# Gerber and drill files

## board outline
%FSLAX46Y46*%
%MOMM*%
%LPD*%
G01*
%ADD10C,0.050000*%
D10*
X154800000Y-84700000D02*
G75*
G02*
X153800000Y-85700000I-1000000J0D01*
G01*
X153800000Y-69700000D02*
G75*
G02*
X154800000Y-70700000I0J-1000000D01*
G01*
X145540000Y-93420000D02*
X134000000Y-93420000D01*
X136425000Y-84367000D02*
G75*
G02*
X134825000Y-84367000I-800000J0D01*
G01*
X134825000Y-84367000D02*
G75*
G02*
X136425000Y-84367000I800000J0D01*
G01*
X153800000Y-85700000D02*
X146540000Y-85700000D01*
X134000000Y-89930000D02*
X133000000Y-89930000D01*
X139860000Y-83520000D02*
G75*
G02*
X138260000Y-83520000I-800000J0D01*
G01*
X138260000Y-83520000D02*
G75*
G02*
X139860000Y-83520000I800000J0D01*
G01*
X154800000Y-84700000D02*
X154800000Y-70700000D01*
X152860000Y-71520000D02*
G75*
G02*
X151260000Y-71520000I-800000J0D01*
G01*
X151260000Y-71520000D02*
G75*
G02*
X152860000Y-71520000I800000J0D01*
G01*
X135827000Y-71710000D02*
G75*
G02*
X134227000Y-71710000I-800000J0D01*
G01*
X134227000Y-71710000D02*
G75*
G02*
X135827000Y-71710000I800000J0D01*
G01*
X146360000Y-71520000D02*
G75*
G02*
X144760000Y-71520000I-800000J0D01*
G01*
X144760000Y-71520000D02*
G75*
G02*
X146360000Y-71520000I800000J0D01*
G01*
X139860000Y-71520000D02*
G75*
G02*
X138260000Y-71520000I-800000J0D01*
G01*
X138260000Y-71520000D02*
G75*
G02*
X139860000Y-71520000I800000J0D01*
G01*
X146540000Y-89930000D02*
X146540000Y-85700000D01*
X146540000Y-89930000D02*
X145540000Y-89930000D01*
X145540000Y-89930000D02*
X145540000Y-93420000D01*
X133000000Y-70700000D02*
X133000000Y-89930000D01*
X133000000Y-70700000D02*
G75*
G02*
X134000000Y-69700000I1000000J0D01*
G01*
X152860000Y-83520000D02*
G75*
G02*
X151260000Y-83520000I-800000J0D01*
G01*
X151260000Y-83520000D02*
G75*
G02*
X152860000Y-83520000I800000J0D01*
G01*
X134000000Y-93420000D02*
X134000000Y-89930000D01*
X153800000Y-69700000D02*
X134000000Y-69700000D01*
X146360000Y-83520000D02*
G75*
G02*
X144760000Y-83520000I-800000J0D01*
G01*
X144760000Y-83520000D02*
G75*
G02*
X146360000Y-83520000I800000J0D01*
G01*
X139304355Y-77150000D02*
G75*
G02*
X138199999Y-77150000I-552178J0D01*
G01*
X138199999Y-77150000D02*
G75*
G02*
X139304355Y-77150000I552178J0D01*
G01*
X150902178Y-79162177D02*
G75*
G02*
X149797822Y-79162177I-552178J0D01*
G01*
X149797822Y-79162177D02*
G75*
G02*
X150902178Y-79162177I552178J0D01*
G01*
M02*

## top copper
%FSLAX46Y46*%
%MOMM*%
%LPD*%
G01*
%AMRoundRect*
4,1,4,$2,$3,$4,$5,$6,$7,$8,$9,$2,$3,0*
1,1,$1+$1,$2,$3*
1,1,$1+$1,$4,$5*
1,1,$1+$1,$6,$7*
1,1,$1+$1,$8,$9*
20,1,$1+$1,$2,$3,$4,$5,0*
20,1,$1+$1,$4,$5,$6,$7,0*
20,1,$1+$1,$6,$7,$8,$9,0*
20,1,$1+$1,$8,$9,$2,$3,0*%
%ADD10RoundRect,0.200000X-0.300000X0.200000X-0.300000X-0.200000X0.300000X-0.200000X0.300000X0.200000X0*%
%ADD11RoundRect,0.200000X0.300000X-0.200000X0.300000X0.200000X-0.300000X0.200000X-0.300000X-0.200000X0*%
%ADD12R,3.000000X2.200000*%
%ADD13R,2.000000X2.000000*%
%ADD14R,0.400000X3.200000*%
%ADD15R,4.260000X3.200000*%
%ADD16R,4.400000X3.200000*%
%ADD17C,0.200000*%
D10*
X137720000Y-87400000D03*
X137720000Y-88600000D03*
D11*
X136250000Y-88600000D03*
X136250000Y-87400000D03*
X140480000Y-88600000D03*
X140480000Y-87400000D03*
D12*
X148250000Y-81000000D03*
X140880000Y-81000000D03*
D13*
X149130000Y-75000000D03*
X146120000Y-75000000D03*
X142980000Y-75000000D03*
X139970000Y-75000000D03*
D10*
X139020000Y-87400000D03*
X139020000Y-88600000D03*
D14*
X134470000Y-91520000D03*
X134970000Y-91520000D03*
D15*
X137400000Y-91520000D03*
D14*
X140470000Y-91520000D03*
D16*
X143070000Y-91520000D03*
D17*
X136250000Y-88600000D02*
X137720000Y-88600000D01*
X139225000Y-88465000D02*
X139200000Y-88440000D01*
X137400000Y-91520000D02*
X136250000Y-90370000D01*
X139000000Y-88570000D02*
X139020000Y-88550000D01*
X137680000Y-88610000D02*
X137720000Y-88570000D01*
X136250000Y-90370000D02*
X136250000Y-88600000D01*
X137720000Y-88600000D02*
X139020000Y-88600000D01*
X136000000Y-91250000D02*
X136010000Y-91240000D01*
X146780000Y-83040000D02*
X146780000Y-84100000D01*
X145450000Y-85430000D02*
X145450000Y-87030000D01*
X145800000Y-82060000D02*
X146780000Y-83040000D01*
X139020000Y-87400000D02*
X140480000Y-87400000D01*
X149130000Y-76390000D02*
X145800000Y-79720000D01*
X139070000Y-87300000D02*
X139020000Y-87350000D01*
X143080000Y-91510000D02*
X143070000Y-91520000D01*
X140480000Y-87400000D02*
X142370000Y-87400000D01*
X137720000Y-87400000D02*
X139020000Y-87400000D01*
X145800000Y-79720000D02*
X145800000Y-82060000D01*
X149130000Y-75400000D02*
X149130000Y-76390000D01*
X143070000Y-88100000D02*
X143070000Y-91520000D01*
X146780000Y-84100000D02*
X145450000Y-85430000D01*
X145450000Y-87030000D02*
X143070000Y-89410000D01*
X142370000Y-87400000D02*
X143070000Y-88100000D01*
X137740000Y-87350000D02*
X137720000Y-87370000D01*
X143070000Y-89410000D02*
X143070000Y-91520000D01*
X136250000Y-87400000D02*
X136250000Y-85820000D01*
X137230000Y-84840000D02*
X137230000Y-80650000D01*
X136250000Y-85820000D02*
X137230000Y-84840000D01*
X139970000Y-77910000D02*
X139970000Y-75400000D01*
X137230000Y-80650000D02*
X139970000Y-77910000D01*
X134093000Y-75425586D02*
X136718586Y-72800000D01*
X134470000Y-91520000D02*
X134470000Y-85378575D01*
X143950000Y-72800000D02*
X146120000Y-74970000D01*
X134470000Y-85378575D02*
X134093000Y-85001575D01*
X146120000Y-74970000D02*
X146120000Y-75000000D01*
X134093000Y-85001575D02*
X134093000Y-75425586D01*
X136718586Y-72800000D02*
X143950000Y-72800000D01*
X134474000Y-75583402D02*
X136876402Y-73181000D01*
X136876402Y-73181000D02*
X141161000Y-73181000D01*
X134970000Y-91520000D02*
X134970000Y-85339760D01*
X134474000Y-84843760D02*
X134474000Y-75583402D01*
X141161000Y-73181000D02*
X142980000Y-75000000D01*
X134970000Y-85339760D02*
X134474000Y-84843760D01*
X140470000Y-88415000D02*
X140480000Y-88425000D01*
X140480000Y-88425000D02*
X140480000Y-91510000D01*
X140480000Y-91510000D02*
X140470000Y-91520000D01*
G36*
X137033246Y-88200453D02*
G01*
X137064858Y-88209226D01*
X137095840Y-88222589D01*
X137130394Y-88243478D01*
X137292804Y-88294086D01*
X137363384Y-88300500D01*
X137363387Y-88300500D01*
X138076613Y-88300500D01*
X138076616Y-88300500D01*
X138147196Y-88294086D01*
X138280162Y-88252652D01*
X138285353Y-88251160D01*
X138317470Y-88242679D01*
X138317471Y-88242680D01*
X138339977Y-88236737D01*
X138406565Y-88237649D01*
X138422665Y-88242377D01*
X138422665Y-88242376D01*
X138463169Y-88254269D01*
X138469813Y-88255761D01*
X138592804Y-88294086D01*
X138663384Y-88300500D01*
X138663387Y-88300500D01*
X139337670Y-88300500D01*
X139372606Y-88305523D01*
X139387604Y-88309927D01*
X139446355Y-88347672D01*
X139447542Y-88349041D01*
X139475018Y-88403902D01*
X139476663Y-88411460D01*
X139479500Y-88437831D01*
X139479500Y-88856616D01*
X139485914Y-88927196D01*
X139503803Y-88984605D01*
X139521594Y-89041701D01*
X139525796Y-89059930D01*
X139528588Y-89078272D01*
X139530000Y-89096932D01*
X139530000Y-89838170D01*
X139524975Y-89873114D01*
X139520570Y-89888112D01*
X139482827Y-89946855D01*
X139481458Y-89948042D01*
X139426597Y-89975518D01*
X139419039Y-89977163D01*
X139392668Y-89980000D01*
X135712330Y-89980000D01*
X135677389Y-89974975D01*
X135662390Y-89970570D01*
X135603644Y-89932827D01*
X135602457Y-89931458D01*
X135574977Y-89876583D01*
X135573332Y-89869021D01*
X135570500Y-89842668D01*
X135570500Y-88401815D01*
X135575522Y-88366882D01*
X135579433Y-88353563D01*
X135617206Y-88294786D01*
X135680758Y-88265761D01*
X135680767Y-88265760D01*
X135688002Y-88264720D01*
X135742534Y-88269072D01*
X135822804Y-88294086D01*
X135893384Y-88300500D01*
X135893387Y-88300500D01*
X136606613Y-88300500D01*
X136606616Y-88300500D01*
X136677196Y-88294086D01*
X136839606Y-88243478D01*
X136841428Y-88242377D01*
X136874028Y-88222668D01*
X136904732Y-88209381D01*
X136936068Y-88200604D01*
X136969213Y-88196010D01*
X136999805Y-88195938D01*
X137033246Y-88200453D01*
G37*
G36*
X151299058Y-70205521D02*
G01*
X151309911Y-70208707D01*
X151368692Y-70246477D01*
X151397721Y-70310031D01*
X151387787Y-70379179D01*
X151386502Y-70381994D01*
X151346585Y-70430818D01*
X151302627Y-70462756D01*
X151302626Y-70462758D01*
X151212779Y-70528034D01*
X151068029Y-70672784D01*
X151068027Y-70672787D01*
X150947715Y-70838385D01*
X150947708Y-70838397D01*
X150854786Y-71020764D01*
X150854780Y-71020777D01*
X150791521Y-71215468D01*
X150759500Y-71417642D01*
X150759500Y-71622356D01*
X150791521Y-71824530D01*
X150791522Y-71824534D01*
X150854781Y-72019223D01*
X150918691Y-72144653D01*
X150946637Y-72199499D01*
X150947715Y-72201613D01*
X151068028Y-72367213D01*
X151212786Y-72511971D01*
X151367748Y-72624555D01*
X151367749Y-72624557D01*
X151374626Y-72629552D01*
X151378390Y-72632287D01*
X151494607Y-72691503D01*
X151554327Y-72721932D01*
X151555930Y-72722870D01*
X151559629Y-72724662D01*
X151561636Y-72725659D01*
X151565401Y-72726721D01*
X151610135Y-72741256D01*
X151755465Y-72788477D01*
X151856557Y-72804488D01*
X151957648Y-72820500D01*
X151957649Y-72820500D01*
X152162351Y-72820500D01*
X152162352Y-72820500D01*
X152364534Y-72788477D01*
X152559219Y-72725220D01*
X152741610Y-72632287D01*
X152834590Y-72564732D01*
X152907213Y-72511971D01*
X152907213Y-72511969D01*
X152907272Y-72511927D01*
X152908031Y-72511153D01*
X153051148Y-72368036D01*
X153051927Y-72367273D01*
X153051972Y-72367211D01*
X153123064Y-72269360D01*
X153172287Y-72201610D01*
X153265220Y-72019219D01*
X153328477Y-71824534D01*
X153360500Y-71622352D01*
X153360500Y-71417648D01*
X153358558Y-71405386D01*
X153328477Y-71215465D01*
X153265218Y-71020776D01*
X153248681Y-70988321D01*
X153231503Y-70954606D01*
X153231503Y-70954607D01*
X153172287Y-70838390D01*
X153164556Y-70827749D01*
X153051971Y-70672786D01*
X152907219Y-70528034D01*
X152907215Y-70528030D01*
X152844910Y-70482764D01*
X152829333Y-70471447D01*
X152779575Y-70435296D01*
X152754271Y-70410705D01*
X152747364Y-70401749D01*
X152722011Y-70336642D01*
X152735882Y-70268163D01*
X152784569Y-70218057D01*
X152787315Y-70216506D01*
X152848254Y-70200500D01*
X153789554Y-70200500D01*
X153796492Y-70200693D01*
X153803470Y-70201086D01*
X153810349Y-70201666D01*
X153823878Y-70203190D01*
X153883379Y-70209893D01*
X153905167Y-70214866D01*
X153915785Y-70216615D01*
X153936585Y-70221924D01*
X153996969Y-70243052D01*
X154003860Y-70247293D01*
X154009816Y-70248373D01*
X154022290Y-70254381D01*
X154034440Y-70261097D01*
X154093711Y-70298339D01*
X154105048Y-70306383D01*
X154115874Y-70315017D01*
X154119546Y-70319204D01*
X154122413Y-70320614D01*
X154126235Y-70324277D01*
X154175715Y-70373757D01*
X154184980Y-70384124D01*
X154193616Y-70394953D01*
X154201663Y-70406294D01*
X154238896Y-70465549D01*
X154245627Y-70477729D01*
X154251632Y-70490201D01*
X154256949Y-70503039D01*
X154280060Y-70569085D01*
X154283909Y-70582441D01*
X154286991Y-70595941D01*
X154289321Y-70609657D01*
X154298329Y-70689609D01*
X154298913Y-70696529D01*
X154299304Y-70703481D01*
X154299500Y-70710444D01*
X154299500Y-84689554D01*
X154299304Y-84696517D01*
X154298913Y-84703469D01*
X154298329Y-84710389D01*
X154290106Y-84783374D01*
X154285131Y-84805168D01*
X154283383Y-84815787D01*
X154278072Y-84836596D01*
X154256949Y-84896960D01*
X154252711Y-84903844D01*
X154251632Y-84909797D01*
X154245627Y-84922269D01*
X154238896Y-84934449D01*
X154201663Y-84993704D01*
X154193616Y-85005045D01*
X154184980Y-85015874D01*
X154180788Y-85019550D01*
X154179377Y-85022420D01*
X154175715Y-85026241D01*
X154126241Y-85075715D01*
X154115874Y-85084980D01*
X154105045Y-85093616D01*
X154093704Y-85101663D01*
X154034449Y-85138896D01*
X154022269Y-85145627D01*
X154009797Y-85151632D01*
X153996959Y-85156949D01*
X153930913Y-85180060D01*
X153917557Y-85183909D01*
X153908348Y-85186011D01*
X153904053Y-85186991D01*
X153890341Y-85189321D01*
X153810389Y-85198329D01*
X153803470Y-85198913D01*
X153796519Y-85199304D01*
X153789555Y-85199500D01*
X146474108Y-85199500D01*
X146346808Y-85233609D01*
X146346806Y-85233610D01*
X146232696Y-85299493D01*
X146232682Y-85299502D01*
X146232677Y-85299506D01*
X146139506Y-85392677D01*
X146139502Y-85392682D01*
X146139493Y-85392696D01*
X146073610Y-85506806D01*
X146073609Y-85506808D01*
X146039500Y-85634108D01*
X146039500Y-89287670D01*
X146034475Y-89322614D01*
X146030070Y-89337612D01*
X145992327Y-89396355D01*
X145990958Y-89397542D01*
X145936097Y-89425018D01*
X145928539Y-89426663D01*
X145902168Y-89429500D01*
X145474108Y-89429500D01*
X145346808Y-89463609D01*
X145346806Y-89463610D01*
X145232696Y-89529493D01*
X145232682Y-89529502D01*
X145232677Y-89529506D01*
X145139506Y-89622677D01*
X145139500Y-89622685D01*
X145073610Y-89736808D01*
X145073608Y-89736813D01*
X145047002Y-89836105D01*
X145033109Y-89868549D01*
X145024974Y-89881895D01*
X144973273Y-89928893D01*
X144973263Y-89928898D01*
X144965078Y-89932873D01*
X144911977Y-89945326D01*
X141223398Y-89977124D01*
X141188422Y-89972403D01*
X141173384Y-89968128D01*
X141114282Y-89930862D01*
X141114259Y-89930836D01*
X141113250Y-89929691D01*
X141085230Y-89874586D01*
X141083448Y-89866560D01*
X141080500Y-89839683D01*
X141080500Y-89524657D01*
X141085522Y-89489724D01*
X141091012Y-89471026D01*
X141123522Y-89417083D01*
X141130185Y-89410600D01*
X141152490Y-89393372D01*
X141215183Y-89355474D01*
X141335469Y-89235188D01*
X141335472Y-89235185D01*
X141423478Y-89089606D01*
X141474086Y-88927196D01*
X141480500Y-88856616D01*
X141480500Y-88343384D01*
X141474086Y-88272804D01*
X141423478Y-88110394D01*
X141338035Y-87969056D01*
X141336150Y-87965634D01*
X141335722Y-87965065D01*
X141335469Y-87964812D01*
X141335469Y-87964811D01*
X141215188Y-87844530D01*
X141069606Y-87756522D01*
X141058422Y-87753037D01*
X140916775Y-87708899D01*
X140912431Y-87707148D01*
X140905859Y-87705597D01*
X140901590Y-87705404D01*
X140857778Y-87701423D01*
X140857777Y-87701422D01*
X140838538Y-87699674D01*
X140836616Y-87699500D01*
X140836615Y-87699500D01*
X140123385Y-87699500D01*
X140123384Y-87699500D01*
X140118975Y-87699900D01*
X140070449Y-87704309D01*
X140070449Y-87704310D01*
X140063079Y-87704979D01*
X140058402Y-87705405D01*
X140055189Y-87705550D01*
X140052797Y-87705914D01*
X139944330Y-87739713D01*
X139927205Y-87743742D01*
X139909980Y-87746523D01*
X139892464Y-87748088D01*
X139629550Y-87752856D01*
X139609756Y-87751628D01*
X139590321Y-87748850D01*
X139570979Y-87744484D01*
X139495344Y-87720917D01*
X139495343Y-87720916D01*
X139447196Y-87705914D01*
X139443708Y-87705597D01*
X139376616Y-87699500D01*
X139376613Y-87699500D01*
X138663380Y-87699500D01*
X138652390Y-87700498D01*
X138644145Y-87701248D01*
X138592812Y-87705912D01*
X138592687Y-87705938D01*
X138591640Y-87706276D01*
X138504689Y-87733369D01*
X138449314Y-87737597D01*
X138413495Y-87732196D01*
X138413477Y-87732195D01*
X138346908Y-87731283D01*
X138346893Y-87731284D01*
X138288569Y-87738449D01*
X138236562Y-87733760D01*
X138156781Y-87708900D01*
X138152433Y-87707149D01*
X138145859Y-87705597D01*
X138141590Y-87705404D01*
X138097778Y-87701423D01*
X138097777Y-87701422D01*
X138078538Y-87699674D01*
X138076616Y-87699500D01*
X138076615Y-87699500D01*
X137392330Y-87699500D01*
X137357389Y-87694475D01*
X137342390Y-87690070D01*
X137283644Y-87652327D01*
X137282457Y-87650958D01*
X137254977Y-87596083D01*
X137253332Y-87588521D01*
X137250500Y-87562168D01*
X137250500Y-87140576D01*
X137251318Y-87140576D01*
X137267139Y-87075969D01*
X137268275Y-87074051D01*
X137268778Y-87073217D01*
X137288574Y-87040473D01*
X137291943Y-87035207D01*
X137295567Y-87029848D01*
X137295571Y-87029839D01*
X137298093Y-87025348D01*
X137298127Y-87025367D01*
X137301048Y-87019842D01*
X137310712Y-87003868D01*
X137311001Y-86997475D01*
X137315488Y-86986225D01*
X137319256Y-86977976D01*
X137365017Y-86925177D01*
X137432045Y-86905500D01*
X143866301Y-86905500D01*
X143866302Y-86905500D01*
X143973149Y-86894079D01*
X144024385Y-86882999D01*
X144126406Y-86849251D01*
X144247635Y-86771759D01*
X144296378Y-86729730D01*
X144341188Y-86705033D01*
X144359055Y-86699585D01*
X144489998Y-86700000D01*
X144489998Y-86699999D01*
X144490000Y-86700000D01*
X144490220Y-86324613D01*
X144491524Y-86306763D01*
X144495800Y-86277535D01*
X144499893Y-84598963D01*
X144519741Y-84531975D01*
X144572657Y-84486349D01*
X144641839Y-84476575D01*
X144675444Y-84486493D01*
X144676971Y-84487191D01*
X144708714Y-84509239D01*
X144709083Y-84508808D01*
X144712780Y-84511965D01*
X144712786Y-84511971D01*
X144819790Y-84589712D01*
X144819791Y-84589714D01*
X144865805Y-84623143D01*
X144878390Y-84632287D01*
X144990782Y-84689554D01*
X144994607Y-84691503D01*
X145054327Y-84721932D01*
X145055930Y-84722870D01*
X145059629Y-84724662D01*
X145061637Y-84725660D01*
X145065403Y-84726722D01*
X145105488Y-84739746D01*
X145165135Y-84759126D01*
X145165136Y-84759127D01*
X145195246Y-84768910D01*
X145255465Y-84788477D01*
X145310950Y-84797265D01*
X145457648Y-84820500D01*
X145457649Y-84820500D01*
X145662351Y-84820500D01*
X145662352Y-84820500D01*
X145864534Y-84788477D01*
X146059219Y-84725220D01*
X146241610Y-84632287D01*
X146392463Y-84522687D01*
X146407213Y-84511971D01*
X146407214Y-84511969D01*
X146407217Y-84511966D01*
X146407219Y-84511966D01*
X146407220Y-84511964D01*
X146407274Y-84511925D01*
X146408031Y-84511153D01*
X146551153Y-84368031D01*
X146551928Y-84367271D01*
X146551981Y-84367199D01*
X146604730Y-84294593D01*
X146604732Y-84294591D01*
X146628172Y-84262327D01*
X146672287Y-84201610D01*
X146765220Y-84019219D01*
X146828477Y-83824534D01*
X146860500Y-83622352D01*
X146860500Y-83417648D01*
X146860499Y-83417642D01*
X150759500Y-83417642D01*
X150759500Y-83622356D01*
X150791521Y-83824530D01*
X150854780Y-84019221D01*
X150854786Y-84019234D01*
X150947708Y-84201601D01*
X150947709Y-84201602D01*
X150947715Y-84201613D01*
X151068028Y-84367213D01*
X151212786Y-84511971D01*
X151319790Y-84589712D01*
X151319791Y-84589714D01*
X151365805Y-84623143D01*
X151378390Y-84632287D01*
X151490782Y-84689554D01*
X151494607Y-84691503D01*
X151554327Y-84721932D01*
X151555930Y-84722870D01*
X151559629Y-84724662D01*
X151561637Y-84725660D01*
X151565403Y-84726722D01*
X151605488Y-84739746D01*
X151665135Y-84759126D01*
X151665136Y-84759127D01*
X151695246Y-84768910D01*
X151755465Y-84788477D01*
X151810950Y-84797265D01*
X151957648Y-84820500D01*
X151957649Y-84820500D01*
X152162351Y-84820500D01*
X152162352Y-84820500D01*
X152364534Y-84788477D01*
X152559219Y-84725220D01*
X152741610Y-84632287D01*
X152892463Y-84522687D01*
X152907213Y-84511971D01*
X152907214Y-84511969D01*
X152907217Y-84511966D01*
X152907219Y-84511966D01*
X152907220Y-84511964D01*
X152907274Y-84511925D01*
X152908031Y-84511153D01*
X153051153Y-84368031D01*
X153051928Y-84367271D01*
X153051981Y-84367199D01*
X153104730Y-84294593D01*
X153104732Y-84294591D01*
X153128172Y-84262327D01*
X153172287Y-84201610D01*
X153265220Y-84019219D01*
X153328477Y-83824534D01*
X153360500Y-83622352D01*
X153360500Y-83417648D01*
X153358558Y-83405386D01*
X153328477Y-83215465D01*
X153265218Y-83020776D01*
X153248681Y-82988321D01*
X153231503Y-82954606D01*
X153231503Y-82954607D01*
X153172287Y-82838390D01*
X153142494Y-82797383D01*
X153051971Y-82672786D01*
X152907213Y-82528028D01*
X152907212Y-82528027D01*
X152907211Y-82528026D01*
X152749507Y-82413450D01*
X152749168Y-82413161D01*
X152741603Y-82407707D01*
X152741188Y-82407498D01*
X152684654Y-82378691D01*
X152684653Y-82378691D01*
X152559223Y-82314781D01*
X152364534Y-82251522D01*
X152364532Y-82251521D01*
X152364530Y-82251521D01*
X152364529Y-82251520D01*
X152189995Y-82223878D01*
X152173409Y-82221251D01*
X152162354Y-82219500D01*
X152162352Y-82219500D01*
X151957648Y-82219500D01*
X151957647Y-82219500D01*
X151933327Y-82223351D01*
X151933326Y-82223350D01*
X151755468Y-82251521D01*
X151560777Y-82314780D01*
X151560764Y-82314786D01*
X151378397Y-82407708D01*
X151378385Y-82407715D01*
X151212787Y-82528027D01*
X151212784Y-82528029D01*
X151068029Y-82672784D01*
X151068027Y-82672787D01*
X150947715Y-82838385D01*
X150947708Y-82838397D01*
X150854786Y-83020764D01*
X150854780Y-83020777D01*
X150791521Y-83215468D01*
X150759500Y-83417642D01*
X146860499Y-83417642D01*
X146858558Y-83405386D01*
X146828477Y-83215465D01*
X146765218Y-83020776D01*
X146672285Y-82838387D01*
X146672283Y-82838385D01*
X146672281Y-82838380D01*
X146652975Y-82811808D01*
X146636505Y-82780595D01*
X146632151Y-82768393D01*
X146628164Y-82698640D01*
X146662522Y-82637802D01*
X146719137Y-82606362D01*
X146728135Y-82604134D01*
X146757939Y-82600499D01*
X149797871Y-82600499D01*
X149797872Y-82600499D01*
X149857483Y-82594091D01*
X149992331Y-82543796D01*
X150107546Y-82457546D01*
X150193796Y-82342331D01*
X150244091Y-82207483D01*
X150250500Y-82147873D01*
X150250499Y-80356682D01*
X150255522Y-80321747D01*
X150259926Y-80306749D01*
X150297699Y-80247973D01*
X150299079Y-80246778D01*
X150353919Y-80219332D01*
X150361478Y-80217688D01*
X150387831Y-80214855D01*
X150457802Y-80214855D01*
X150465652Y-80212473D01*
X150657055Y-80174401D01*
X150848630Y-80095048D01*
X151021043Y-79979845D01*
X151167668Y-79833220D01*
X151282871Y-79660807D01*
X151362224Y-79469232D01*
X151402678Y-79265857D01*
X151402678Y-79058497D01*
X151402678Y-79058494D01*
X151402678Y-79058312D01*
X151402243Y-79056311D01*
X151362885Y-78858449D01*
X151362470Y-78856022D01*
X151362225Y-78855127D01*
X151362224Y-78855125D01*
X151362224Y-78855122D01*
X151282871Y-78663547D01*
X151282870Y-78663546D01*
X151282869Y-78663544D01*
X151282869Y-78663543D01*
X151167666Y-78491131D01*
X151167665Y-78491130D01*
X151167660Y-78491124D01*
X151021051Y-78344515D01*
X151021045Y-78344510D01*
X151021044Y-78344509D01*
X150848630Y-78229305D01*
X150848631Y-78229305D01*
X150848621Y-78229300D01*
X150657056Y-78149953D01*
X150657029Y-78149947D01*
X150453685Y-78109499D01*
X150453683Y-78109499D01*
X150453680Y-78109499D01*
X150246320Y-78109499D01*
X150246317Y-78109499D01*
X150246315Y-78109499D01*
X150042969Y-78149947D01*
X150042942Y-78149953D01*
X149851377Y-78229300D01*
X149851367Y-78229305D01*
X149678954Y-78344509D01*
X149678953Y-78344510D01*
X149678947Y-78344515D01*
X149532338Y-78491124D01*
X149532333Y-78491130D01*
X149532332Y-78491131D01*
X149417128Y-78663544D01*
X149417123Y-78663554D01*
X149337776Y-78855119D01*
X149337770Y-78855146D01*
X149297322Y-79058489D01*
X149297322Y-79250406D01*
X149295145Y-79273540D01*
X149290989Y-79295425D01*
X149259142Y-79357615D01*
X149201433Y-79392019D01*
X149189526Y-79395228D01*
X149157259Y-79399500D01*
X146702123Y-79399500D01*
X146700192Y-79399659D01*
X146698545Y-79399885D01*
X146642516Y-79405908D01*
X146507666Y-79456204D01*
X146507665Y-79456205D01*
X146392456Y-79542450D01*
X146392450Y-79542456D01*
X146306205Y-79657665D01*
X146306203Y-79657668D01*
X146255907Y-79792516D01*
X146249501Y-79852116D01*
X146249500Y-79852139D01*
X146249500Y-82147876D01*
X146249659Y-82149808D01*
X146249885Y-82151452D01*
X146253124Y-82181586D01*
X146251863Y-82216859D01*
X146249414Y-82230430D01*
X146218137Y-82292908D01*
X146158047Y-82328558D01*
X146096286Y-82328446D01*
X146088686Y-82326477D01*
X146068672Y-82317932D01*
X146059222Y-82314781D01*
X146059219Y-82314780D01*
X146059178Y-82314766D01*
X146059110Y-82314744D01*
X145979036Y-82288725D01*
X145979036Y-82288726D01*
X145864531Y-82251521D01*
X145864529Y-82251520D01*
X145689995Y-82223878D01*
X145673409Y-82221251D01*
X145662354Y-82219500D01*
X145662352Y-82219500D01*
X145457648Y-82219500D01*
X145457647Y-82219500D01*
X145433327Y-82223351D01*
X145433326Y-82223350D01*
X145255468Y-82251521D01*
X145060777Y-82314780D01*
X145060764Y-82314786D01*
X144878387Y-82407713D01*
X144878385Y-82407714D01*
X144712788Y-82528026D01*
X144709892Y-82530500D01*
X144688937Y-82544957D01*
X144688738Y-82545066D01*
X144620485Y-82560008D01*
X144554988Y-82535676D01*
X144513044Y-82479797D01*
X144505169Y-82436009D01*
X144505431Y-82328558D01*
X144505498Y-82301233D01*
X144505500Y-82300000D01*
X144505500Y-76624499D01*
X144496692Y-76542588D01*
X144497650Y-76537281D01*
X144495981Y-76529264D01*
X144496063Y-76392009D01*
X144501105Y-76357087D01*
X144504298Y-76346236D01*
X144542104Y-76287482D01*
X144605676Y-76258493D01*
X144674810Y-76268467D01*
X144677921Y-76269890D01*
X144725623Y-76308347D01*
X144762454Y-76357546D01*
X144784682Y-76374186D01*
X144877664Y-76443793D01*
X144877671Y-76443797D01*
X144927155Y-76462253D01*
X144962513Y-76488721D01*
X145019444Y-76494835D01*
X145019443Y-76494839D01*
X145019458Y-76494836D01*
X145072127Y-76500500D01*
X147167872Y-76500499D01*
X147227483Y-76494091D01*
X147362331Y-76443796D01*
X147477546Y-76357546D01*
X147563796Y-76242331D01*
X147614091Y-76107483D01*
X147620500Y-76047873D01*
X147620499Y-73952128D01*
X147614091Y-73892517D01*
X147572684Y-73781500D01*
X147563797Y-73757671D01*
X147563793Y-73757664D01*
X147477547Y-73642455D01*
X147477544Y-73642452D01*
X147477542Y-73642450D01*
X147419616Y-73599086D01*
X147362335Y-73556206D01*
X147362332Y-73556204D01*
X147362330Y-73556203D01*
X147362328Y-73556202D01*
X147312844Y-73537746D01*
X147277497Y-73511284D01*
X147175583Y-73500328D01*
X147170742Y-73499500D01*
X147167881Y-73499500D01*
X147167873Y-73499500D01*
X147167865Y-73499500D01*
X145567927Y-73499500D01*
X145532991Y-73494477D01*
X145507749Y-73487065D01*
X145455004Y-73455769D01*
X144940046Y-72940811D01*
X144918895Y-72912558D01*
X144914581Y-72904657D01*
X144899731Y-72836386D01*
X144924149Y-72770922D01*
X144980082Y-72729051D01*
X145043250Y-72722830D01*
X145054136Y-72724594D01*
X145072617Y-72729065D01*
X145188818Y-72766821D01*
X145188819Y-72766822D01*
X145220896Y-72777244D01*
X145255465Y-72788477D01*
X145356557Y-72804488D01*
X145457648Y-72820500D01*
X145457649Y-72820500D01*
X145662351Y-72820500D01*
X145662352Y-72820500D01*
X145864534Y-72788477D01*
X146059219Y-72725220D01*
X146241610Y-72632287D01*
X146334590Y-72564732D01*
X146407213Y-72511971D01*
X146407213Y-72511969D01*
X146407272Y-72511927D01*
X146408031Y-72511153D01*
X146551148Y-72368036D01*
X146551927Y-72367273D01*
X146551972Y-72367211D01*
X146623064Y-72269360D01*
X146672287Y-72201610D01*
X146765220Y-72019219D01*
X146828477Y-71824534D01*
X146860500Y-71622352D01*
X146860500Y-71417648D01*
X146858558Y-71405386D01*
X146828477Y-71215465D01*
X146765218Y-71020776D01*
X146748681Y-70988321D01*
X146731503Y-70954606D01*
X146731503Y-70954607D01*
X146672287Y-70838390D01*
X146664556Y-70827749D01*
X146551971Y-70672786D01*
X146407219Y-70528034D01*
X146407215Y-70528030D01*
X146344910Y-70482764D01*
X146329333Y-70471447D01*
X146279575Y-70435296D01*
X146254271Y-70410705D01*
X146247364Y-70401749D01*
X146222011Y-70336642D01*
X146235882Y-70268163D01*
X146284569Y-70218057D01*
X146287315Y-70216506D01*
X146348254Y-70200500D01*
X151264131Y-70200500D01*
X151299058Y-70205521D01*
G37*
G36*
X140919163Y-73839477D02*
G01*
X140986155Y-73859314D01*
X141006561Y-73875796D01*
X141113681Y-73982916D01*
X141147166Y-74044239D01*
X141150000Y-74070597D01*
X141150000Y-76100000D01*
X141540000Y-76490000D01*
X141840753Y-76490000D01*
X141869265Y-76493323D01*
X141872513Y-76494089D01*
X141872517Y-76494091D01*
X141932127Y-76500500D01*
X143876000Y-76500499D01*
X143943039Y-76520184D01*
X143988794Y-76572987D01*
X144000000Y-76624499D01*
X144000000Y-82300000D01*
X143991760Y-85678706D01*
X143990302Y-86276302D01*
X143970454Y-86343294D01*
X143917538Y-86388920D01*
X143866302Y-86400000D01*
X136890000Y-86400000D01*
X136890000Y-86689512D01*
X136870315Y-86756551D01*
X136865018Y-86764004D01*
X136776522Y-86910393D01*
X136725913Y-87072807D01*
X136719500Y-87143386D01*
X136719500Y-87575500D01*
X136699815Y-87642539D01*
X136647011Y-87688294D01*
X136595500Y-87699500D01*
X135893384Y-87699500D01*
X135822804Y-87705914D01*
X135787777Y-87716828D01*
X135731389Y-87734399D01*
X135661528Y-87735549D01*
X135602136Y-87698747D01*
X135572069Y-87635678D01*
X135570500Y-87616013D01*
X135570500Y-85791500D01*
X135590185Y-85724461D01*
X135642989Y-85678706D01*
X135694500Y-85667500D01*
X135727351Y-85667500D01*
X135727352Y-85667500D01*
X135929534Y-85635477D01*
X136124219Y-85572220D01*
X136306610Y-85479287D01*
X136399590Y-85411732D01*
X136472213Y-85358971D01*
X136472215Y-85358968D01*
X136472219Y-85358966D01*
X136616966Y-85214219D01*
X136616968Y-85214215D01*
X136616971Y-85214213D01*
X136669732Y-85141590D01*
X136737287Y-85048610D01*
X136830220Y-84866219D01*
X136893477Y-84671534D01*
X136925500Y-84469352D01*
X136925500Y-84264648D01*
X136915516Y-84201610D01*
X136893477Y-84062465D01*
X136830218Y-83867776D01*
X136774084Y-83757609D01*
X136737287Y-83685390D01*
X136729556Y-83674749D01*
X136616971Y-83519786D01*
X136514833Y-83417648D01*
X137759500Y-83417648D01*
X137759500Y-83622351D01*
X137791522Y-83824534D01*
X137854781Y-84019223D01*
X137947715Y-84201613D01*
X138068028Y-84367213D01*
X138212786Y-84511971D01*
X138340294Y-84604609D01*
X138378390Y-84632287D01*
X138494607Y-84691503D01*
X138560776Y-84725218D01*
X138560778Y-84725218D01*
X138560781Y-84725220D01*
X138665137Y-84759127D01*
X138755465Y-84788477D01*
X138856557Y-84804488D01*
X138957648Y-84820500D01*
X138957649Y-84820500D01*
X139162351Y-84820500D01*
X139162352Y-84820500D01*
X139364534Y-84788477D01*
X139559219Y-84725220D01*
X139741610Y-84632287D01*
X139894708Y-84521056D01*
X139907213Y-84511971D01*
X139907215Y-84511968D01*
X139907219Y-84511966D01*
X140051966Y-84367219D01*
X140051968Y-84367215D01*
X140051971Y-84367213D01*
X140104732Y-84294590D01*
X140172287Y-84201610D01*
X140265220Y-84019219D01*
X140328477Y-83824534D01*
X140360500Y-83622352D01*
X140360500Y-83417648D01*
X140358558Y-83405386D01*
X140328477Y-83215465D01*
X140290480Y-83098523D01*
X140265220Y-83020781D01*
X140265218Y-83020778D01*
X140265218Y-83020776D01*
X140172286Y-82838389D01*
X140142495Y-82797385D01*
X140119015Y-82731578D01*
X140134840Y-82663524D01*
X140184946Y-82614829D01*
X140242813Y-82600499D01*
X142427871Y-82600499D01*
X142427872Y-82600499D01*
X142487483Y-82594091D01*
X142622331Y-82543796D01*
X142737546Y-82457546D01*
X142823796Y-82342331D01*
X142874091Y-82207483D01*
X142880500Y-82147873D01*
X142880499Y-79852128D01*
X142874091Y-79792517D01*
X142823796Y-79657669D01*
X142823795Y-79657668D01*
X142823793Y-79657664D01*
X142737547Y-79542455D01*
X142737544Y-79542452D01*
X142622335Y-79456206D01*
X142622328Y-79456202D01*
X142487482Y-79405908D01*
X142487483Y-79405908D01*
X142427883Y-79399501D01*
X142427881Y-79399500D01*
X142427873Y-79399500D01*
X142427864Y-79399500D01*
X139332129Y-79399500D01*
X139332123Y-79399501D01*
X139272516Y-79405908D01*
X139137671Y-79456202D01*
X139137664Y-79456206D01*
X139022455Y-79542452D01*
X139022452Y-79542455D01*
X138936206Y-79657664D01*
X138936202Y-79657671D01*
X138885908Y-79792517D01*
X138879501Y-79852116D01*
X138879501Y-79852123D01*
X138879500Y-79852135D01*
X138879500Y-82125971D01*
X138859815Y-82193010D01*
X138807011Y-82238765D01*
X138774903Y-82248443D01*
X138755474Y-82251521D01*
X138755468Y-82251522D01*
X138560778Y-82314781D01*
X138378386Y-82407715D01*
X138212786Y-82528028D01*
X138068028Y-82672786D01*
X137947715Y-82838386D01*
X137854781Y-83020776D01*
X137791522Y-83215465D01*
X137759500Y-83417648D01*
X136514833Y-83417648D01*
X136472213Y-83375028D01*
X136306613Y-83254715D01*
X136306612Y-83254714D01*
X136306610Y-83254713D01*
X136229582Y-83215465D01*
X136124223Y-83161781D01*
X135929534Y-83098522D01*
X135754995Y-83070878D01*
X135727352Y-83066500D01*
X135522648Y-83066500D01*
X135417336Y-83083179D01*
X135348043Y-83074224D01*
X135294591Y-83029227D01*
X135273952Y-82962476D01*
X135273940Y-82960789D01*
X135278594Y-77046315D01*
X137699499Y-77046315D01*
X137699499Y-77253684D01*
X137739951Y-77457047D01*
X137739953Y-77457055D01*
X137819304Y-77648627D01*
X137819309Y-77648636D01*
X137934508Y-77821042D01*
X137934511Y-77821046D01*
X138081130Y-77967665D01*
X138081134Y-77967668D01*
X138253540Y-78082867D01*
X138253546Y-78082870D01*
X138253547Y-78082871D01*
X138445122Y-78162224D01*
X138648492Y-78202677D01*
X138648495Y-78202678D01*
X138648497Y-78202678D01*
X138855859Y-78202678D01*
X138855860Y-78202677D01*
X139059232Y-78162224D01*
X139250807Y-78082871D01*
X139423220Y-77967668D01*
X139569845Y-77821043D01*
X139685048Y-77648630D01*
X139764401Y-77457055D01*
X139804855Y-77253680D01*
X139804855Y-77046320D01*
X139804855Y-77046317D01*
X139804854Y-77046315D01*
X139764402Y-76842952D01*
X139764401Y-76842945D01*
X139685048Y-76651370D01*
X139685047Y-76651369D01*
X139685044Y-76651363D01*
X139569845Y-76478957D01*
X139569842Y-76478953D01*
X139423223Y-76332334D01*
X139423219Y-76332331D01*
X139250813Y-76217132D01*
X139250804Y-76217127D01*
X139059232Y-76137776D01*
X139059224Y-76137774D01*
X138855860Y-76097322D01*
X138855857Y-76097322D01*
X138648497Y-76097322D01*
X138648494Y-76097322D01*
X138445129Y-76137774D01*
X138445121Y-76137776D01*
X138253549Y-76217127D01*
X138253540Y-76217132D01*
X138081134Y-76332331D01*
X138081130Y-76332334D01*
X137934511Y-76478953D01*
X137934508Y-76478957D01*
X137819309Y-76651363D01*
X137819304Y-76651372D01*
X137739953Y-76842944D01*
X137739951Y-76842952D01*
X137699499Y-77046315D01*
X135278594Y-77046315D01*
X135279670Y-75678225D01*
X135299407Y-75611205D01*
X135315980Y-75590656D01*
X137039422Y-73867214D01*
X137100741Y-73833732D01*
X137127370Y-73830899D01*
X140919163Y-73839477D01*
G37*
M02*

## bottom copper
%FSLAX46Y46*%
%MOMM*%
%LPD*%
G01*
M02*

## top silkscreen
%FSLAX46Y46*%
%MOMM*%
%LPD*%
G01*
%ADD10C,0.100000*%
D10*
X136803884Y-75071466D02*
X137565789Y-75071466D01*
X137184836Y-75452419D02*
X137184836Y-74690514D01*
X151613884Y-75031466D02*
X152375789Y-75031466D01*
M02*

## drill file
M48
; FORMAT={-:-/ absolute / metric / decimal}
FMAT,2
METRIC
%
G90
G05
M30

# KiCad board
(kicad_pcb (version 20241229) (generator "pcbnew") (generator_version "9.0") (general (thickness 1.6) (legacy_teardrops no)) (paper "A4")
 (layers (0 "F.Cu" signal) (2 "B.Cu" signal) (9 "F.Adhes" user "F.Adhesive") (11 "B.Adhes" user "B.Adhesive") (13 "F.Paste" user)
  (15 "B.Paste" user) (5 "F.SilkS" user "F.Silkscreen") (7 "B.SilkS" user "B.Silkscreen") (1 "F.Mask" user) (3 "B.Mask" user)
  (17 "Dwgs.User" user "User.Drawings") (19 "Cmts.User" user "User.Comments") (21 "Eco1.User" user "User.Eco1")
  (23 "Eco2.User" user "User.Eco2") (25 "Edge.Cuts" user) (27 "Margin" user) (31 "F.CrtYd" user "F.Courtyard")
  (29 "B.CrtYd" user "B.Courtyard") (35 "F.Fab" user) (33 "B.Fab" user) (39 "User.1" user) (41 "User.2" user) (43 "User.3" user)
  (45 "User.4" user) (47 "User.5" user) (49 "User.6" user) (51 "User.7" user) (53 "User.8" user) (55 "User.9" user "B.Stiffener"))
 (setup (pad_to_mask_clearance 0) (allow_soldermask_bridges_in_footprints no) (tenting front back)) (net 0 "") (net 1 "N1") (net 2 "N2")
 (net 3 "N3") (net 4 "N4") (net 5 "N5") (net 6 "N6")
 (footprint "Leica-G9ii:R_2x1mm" (layer "F.Cu") (at 137.72 88 -90)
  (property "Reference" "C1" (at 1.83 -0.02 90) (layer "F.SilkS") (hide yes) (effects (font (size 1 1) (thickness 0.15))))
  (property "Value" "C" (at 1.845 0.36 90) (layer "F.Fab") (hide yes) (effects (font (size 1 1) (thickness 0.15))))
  (pad "1" smd roundrect (at -0.6 0 270) (size 0.8 1) (layers "F.Cu" "F.Mask" "F.Paste") (roundrect_rratio 0.25) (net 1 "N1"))
  (pad "2" smd roundrect (at 0.6 0 270) (size 0.8 1) (layers "F.Cu" "F.Mask" "F.Paste") (roundrect_rratio 0.25) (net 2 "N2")))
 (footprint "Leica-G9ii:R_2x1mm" (layer "F.Cu") (at 136.25 88 90)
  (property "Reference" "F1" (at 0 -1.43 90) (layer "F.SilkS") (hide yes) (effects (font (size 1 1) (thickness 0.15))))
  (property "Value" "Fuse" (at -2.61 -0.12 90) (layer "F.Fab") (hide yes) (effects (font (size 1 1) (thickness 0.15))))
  (pad "1" smd roundrect (at -0.6 0 90) (size 0.8 1) (layers "F.Cu" "F.Mask" "F.Paste") (roundrect_rratio 0.25) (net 2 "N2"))
  (pad "2" smd roundrect (at 0.6 0 90) (size 0.8 1) (layers "F.Cu" "F.Mask" "F.Paste") (roundrect_rratio 0.25) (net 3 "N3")))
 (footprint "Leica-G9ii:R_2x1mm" (layer "F.Cu") (at 140.48 88 90)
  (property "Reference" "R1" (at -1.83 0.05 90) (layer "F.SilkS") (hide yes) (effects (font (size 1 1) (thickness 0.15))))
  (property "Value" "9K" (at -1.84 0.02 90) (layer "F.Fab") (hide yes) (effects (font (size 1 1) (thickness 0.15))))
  (pad "1" smd roundrect (at -0.6 0 90) (size 0.8 1) (layers "F.Cu" "F.Mask" "F.Paste") (roundrect_rratio 0.25) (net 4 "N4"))
  (pad "2" smd roundrect (at 0.6 0 90) (size 0.8 1) (layers "F.Cu" "F.Mask" "F.Paste") (roundrect_rratio 0.25) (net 1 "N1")))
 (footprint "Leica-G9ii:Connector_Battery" (layer "F.Cu") (at 144.55 78 180)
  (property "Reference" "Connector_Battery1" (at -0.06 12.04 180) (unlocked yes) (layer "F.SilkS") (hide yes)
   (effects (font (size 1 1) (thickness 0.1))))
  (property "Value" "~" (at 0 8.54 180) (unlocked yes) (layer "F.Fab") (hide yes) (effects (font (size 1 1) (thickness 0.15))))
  (fp_circle (center 5.797823 0.85) (end 6.247823 0.53) (stroke (width 0.05) (type default)) (fill no) (layer "Edge.Cuts"))
  (fp_circle (center -5.8 -1.162177) (end -5.35 -1.482177) (stroke (width 0.05) (type default)) (fill no) (layer "Edge.Cuts"))
  (pad "" smd roundrect (at -4.58 3 180) (size 1.4 1.4) (layers "F.Mask" "F.Paste") (roundrect_rratio 0.125))
  (pad "" smd roundrect (at -3.7 -3 180) (size 1.4 1.4) (layers "F.Mask" "F.Paste") (roundrect_rratio 0.125))
  (pad "" smd rect (at -3.7 -3 180) (size 3 2.2) (layers "F.Cu"))
  (pad "" smd roundrect (at -1.57 3 180) (size 1.4 1.4) (layers "F.Mask" "F.Paste") (roundrect_rratio 0.125))
  (pad "" smd roundrect (at 1.57 3 90) (size 1.4 1.4) (layers "F.Mask" "F.Paste") (roundrect_rratio 0.125))
  (pad "" smd roundrect (at 3.67 -3 180) (size 1.4 1.4) (layers "F.Mask" "F.Paste") (roundrect_rratio 0.125))
  (pad "" smd rect (at 3.67 -3 180) (size 3 2.2) (layers "F.Cu"))
  (pad "" smd roundrect (at 4.58 3 180) (size 1.4 1.4) (layers "F.Mask" "F.Paste") (roundrect_rratio 0.125))
  (pad "1" smd rect (at -4.58 3 180) (size 2 2) (layers "F.Cu") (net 1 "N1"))
  (pad "2" smd rect (at -1.57 3 180) (size 2 2) (layers "F.Cu") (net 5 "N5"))
  (pad "3" smd rect (at 1.57 3 180) (size 2 2) (layers "F.Cu") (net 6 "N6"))
  (pad "4" smd rect (at 4.58 3 180) (size 2 2) (layers "F.Cu") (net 3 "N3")))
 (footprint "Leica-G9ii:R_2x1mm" (layer "F.Cu") (at 139.02 88 -90)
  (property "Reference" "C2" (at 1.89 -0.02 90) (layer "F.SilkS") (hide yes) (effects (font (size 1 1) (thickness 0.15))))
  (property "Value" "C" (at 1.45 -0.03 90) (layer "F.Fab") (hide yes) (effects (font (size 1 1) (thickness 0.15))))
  (pad "1" smd roundrect (at -0.6 0 270) (size 0.8 1) (layers "F.Cu" "F.Mask" "F.Paste") (roundrect_rratio 0.25) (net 1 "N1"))
  (pad "2" smd roundrect (at 0.6 0 270) (size 0.8 1) (layers "F.Cu" "F.Mask" "F.Paste") (roundrect_rratio 0.25) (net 2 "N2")))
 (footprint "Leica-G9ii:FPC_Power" (layer "F.Cu") (at 139.7 91.695)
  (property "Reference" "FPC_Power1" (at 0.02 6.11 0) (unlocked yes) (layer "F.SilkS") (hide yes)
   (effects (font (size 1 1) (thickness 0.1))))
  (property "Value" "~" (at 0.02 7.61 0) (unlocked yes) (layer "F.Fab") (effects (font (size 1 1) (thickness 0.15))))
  (pad "1" connect rect (at -5.23 -0.175) (size 0.4 3.2) (layers "F.Cu" "F.Mask") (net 5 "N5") (clearance 0.05))
  (pad "2" connect rect (at -4.73 -0.175) (size 0.4 3.2) (layers "F.Cu" "F.Mask") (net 6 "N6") (clearance 0.05))
  (pad "3" connect rect (at -2.3 -0.175) (size 4.26 3.2) (layers "F.Cu" "F.Mask") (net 2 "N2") (clearance 0.05))
  (pad "4" connect rect (at 0.77 -0.175) (size 0.4 3.2) (layers "F.Cu" "F.Mask") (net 4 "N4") (clearance 0.05))
  (pad "5" connect rect (at 3.37 -0.175) (size 4.4 3.2) (layers "F.Cu" "F.Mask") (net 1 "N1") (clearance 0.05)))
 (gr_arc (start 154.8 84.7) (mid 154.507107 85.407107) (end 153.8 85.7) (stroke (width 0.05) (type default)) (layer "Edge.Cuts"))
 (gr_arc (start 153.8 69.7) (mid 154.507107 69.992893) (end 154.8 70.7) (stroke (width 0.05) (type default)) (layer "Edge.Cuts"))
 (gr_line (start 145.54 93.42) (end 134 93.42) (stroke (width 0.05) (type default)) (layer "Edge.Cuts"))
 (gr_circle (center 135.625 84.367) (end 136.425 84.367) (stroke (width 0.05) (type solid)) (fill no) (layer "Edge.Cuts"))
 (gr_line (start 153.8 85.7) (end 146.54 85.7) (stroke (width 0.05) (type default)) (layer "Edge.Cuts"))
 (gr_line (start 134 89.93) (end 133 89.93) (stroke (width 0.05) (type default)) (layer "Edge.Cuts"))
 (gr_circle (center 139.06 83.52) (end 139.86 83.52) (stroke (width 0.05) (type default)) (fill no) (layer "Edge.Cuts"))
 (gr_line (start 154.8 84.7) (end 154.8 70.7) (stroke (width 0.05) (type default)) (layer "Edge.Cuts"))
 (gr_circle (center 152.06 71.52) (end 152.86 71.52) (stroke (width 0.05) (type default)) (fill no) (layer "Edge.Cuts"))
 (gr_circle (center 135.027 71.71) (end 135.827 71.71) (stroke (width 0.05) (type solid)) (fill no) (layer "Edge.Cuts"))
 (gr_circle (center 145.56 71.52) (end 146.36 71.52) (stroke (width 0.05) (type default)) (fill no) (layer "Edge.Cuts"))
 (gr_circle (center 139.06 71.52) (end 139.86 71.52) (stroke (width 0.05) (type default)) (fill no) (layer "Edge.Cuts"))
 (gr_line (start 146.54 89.93) (end 146.54 85.7) (stroke (width 0.05) (type default)) (layer "Edge.Cuts"))
 (gr_line (start 146.54 89.93) (end 145.54 89.93) (stroke (width 0.05) (type default)) (layer "Edge.Cuts"))
 (gr_line (start 145.54 89.93) (end 145.54 93.42) (stroke (width 0.05) (type default)) (layer "Edge.Cuts"))
 (gr_line (start 133 70.7) (end 133 89.93) (stroke (width 0.05) (type default)) (layer "Edge.Cuts"))
 (gr_arc (start 133 70.7) (mid 133.292893 69.992893) (end 134 69.7) (stroke (width 0.05) (type default)) (layer "Edge.Cuts"))
 (gr_circle (center 152.06 83.52) (end 152.86 83.52) (stroke (width 0.05) (type default)) (fill no) (layer "Edge.Cuts"))
 (gr_line (start 134 93.42) (end 134 89.93) (stroke (width 0.05) (type default)) (layer "Edge.Cuts"))
 (gr_line (start 153.8 69.7) (end 134 69.7) (stroke (width 0.05) (type default)) (layer "Edge.Cuts"))
 (gr_circle (center 145.56 83.52) (end 146.36 83.52) (stroke (width 0.05) (type default)) (fill no) (layer "Edge.Cuts"))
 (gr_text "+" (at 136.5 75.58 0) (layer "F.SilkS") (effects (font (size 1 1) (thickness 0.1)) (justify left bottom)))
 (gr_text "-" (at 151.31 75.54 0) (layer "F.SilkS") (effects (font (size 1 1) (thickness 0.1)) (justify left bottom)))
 (segment (start 136.25 88.6) (end 137.72 88.6) (width 0.2) (layer "F.Cu") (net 2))
 (segment (start 139.225 88.465) (end 139.2 88.44) (width 0.2) (layer "F.Cu") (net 2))
 (segment (start 137.4 91.52) (end 136.25 90.37) (width 0.2) (layer "F.Cu") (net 2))
 (segment (start 139 88.57) (end 139.02 88.55) (width 0.2) (layer "F.Cu") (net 2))
 (segment (start 137.68 88.61) (end 137.72 88.57) (width 0.2) (layer "F.Cu") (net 2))
 (segment (start 136.25 90.37) (end 136.25 88.6) (width 0.2) (layer "F.Cu") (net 2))
 (segment (start 137.72 88.6) (end 139.02 88.6) (width 0.2) (layer "F.Cu") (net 2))
 (segment (start 136 91.25) (end 136.01 91.24) (width 0.2) (layer "F.Cu") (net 2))
 (segment (start 146.78 83.04) (end 146.78 84.1) (width 0.2) (layer "F.Cu") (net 1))
 (segment (start 145.45 85.43) (end 145.45 87.03) (width 0.2) (layer "F.Cu") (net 1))
 (segment (start 145.8 82.06) (end 146.78 83.04) (width 0.2) (layer "F.Cu") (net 1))
 (segment (start 139.02 87.4) (end 140.48 87.4) (width 0.2) (layer "F.Cu") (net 1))
 (segment (start 149.13 76.39) (end 145.8 79.72) (width 0.2) (layer "F.Cu") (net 1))
 (segment (start 139.07 87.3) (end 139.02 87.35) (width 0.2) (layer "F.Cu") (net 1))
 (segment (start 143.08 91.51) (end 143.07 91.52) (width 0.2) (layer "F.Cu") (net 1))
 (segment (start 140.48 87.4) (end 142.37 87.4) (width 0.2) (layer "F.Cu") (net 1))
 (segment (start 137.72 87.4) (end 139.02 87.4) (width 0.2) (layer "F.Cu") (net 1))
 (segment (start 145.8 79.72) (end 145.8 82.06) (width 0.2) (layer "F.Cu") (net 1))
 (segment (start 149.13 75.4) (end 149.13 76.39) (width 0.2) (layer "F.Cu") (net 1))
 (segment (start 143.07 88.1) (end 143.07 91.52) (width 0.2) (layer "F.Cu") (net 1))
 (segment (start 146.78 84.1) (end 145.45 85.43) (width 0.2) (layer "F.Cu") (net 1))
 (segment (start 145.45 87.03) (end 143.07 89.41) (width 0.2) (layer "F.Cu") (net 1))
 (segment (start 142.37 87.4) (end 143.07 88.1) (width 0.2) (layer "F.Cu") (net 1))
 (segment (start 137.74 87.35) (end 137.72 87.37) (width 0.2) (layer "F.Cu") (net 1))
 (segment (start 143.07 89.41) (end 143.07 91.52) (width 0.2) (layer "F.Cu") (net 1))
 (segment (start 136.25 87.4) (end 136.25 85.82) (width 0.2) (layer "F.Cu") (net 3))
 (segment (start 137.23 84.84) (end 137.23 80.65) (width 0.2) (layer "F.Cu") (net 3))
 (segment (start 136.25 85.82) (end 137.23 84.84) (width 0.2) (layer "F.Cu") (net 3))
 (segment (start 139.97 77.91) (end 139.97 75.4) (width 0.2) (layer "F.Cu") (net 3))
 (segment (start 137.23 80.65) (end 139.97 77.91) (width 0.2) (layer "F.Cu") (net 3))
 (segment (start 134.093 75.425586) (end 136.718586 72.8) (width 0.2) (layer "F.Cu") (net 5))
 (segment (start 134.47 91.52) (end 134.47 85.378575) (width 0.2) (layer "F.Cu") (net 5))
 (segment (start 143.95 72.8) (end 146.12 74.97) (width 0.2) (layer "F.Cu") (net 5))
 (segment (start 134.47 85.378575) (end 134.093 85.001575) (width 0.2) (layer "F.Cu") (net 5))
 (segment (start 146.12 74.97) (end 146.12 75) (width 0.2) (layer "F.Cu") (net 5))
 (segment (start 134.093 85.001575) (end 134.093 75.425586) (width 0.2) (layer "F.Cu") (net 5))
 (segment (start 136.718586 72.8) (end 143.95 72.8) (width 0.2) (layer "F.Cu") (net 5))
 (segment (start 134.474 75.583402) (end 136.876402 73.181) (width 0.2) (layer "F.Cu") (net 6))
 (segment (start 136.876402 73.181) (end 141.161 73.181) (width 0.2) (layer "F.Cu") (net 6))
 (segment (start 134.97 91.52) (end 134.97 85.33976) (width 0.2) (layer "F.Cu") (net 6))
 (segment (start 134.474 84.84376) (end 134.474 75.583402) (width 0.2) (layer "F.Cu") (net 6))
 (segment (start 141.161 73.181) (end 142.98 75) (width 0.2) (layer "F.Cu") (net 6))
 (segment (start 134.97 85.33976) (end 134.474 84.84376) (width 0.2) (layer "F.Cu") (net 6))
 (segment (start 140.47 88.415) (end 140.48 88.425) (width 0.2) (layer "F.Cu") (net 4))
 (segment (start 140.48 88.425) (end 140.48 91.51) (width 0.2) (layer "F.Cu") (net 4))
 (segment (start 140.48 91.51) (end 140.47 91.52) (width 0.2) (layer "F.Cu") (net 4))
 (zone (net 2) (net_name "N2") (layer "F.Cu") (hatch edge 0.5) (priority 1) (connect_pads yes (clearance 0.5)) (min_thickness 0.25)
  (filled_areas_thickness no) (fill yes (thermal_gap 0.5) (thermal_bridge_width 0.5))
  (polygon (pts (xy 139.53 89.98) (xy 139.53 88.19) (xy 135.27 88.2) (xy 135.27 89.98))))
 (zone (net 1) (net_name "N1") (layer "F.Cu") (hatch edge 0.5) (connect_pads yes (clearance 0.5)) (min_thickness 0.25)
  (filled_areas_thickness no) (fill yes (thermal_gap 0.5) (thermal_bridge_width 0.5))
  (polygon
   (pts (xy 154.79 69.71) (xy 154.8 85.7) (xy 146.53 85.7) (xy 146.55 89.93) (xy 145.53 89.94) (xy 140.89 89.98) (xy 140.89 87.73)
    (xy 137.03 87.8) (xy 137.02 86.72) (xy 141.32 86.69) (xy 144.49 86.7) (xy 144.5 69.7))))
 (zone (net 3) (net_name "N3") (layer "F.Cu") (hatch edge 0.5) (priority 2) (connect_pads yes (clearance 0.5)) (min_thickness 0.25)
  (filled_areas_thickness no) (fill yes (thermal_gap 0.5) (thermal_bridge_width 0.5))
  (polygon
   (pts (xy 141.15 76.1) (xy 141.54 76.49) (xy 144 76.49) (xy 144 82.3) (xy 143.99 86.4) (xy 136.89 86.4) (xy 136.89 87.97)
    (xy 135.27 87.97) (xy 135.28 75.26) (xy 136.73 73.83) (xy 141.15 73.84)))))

